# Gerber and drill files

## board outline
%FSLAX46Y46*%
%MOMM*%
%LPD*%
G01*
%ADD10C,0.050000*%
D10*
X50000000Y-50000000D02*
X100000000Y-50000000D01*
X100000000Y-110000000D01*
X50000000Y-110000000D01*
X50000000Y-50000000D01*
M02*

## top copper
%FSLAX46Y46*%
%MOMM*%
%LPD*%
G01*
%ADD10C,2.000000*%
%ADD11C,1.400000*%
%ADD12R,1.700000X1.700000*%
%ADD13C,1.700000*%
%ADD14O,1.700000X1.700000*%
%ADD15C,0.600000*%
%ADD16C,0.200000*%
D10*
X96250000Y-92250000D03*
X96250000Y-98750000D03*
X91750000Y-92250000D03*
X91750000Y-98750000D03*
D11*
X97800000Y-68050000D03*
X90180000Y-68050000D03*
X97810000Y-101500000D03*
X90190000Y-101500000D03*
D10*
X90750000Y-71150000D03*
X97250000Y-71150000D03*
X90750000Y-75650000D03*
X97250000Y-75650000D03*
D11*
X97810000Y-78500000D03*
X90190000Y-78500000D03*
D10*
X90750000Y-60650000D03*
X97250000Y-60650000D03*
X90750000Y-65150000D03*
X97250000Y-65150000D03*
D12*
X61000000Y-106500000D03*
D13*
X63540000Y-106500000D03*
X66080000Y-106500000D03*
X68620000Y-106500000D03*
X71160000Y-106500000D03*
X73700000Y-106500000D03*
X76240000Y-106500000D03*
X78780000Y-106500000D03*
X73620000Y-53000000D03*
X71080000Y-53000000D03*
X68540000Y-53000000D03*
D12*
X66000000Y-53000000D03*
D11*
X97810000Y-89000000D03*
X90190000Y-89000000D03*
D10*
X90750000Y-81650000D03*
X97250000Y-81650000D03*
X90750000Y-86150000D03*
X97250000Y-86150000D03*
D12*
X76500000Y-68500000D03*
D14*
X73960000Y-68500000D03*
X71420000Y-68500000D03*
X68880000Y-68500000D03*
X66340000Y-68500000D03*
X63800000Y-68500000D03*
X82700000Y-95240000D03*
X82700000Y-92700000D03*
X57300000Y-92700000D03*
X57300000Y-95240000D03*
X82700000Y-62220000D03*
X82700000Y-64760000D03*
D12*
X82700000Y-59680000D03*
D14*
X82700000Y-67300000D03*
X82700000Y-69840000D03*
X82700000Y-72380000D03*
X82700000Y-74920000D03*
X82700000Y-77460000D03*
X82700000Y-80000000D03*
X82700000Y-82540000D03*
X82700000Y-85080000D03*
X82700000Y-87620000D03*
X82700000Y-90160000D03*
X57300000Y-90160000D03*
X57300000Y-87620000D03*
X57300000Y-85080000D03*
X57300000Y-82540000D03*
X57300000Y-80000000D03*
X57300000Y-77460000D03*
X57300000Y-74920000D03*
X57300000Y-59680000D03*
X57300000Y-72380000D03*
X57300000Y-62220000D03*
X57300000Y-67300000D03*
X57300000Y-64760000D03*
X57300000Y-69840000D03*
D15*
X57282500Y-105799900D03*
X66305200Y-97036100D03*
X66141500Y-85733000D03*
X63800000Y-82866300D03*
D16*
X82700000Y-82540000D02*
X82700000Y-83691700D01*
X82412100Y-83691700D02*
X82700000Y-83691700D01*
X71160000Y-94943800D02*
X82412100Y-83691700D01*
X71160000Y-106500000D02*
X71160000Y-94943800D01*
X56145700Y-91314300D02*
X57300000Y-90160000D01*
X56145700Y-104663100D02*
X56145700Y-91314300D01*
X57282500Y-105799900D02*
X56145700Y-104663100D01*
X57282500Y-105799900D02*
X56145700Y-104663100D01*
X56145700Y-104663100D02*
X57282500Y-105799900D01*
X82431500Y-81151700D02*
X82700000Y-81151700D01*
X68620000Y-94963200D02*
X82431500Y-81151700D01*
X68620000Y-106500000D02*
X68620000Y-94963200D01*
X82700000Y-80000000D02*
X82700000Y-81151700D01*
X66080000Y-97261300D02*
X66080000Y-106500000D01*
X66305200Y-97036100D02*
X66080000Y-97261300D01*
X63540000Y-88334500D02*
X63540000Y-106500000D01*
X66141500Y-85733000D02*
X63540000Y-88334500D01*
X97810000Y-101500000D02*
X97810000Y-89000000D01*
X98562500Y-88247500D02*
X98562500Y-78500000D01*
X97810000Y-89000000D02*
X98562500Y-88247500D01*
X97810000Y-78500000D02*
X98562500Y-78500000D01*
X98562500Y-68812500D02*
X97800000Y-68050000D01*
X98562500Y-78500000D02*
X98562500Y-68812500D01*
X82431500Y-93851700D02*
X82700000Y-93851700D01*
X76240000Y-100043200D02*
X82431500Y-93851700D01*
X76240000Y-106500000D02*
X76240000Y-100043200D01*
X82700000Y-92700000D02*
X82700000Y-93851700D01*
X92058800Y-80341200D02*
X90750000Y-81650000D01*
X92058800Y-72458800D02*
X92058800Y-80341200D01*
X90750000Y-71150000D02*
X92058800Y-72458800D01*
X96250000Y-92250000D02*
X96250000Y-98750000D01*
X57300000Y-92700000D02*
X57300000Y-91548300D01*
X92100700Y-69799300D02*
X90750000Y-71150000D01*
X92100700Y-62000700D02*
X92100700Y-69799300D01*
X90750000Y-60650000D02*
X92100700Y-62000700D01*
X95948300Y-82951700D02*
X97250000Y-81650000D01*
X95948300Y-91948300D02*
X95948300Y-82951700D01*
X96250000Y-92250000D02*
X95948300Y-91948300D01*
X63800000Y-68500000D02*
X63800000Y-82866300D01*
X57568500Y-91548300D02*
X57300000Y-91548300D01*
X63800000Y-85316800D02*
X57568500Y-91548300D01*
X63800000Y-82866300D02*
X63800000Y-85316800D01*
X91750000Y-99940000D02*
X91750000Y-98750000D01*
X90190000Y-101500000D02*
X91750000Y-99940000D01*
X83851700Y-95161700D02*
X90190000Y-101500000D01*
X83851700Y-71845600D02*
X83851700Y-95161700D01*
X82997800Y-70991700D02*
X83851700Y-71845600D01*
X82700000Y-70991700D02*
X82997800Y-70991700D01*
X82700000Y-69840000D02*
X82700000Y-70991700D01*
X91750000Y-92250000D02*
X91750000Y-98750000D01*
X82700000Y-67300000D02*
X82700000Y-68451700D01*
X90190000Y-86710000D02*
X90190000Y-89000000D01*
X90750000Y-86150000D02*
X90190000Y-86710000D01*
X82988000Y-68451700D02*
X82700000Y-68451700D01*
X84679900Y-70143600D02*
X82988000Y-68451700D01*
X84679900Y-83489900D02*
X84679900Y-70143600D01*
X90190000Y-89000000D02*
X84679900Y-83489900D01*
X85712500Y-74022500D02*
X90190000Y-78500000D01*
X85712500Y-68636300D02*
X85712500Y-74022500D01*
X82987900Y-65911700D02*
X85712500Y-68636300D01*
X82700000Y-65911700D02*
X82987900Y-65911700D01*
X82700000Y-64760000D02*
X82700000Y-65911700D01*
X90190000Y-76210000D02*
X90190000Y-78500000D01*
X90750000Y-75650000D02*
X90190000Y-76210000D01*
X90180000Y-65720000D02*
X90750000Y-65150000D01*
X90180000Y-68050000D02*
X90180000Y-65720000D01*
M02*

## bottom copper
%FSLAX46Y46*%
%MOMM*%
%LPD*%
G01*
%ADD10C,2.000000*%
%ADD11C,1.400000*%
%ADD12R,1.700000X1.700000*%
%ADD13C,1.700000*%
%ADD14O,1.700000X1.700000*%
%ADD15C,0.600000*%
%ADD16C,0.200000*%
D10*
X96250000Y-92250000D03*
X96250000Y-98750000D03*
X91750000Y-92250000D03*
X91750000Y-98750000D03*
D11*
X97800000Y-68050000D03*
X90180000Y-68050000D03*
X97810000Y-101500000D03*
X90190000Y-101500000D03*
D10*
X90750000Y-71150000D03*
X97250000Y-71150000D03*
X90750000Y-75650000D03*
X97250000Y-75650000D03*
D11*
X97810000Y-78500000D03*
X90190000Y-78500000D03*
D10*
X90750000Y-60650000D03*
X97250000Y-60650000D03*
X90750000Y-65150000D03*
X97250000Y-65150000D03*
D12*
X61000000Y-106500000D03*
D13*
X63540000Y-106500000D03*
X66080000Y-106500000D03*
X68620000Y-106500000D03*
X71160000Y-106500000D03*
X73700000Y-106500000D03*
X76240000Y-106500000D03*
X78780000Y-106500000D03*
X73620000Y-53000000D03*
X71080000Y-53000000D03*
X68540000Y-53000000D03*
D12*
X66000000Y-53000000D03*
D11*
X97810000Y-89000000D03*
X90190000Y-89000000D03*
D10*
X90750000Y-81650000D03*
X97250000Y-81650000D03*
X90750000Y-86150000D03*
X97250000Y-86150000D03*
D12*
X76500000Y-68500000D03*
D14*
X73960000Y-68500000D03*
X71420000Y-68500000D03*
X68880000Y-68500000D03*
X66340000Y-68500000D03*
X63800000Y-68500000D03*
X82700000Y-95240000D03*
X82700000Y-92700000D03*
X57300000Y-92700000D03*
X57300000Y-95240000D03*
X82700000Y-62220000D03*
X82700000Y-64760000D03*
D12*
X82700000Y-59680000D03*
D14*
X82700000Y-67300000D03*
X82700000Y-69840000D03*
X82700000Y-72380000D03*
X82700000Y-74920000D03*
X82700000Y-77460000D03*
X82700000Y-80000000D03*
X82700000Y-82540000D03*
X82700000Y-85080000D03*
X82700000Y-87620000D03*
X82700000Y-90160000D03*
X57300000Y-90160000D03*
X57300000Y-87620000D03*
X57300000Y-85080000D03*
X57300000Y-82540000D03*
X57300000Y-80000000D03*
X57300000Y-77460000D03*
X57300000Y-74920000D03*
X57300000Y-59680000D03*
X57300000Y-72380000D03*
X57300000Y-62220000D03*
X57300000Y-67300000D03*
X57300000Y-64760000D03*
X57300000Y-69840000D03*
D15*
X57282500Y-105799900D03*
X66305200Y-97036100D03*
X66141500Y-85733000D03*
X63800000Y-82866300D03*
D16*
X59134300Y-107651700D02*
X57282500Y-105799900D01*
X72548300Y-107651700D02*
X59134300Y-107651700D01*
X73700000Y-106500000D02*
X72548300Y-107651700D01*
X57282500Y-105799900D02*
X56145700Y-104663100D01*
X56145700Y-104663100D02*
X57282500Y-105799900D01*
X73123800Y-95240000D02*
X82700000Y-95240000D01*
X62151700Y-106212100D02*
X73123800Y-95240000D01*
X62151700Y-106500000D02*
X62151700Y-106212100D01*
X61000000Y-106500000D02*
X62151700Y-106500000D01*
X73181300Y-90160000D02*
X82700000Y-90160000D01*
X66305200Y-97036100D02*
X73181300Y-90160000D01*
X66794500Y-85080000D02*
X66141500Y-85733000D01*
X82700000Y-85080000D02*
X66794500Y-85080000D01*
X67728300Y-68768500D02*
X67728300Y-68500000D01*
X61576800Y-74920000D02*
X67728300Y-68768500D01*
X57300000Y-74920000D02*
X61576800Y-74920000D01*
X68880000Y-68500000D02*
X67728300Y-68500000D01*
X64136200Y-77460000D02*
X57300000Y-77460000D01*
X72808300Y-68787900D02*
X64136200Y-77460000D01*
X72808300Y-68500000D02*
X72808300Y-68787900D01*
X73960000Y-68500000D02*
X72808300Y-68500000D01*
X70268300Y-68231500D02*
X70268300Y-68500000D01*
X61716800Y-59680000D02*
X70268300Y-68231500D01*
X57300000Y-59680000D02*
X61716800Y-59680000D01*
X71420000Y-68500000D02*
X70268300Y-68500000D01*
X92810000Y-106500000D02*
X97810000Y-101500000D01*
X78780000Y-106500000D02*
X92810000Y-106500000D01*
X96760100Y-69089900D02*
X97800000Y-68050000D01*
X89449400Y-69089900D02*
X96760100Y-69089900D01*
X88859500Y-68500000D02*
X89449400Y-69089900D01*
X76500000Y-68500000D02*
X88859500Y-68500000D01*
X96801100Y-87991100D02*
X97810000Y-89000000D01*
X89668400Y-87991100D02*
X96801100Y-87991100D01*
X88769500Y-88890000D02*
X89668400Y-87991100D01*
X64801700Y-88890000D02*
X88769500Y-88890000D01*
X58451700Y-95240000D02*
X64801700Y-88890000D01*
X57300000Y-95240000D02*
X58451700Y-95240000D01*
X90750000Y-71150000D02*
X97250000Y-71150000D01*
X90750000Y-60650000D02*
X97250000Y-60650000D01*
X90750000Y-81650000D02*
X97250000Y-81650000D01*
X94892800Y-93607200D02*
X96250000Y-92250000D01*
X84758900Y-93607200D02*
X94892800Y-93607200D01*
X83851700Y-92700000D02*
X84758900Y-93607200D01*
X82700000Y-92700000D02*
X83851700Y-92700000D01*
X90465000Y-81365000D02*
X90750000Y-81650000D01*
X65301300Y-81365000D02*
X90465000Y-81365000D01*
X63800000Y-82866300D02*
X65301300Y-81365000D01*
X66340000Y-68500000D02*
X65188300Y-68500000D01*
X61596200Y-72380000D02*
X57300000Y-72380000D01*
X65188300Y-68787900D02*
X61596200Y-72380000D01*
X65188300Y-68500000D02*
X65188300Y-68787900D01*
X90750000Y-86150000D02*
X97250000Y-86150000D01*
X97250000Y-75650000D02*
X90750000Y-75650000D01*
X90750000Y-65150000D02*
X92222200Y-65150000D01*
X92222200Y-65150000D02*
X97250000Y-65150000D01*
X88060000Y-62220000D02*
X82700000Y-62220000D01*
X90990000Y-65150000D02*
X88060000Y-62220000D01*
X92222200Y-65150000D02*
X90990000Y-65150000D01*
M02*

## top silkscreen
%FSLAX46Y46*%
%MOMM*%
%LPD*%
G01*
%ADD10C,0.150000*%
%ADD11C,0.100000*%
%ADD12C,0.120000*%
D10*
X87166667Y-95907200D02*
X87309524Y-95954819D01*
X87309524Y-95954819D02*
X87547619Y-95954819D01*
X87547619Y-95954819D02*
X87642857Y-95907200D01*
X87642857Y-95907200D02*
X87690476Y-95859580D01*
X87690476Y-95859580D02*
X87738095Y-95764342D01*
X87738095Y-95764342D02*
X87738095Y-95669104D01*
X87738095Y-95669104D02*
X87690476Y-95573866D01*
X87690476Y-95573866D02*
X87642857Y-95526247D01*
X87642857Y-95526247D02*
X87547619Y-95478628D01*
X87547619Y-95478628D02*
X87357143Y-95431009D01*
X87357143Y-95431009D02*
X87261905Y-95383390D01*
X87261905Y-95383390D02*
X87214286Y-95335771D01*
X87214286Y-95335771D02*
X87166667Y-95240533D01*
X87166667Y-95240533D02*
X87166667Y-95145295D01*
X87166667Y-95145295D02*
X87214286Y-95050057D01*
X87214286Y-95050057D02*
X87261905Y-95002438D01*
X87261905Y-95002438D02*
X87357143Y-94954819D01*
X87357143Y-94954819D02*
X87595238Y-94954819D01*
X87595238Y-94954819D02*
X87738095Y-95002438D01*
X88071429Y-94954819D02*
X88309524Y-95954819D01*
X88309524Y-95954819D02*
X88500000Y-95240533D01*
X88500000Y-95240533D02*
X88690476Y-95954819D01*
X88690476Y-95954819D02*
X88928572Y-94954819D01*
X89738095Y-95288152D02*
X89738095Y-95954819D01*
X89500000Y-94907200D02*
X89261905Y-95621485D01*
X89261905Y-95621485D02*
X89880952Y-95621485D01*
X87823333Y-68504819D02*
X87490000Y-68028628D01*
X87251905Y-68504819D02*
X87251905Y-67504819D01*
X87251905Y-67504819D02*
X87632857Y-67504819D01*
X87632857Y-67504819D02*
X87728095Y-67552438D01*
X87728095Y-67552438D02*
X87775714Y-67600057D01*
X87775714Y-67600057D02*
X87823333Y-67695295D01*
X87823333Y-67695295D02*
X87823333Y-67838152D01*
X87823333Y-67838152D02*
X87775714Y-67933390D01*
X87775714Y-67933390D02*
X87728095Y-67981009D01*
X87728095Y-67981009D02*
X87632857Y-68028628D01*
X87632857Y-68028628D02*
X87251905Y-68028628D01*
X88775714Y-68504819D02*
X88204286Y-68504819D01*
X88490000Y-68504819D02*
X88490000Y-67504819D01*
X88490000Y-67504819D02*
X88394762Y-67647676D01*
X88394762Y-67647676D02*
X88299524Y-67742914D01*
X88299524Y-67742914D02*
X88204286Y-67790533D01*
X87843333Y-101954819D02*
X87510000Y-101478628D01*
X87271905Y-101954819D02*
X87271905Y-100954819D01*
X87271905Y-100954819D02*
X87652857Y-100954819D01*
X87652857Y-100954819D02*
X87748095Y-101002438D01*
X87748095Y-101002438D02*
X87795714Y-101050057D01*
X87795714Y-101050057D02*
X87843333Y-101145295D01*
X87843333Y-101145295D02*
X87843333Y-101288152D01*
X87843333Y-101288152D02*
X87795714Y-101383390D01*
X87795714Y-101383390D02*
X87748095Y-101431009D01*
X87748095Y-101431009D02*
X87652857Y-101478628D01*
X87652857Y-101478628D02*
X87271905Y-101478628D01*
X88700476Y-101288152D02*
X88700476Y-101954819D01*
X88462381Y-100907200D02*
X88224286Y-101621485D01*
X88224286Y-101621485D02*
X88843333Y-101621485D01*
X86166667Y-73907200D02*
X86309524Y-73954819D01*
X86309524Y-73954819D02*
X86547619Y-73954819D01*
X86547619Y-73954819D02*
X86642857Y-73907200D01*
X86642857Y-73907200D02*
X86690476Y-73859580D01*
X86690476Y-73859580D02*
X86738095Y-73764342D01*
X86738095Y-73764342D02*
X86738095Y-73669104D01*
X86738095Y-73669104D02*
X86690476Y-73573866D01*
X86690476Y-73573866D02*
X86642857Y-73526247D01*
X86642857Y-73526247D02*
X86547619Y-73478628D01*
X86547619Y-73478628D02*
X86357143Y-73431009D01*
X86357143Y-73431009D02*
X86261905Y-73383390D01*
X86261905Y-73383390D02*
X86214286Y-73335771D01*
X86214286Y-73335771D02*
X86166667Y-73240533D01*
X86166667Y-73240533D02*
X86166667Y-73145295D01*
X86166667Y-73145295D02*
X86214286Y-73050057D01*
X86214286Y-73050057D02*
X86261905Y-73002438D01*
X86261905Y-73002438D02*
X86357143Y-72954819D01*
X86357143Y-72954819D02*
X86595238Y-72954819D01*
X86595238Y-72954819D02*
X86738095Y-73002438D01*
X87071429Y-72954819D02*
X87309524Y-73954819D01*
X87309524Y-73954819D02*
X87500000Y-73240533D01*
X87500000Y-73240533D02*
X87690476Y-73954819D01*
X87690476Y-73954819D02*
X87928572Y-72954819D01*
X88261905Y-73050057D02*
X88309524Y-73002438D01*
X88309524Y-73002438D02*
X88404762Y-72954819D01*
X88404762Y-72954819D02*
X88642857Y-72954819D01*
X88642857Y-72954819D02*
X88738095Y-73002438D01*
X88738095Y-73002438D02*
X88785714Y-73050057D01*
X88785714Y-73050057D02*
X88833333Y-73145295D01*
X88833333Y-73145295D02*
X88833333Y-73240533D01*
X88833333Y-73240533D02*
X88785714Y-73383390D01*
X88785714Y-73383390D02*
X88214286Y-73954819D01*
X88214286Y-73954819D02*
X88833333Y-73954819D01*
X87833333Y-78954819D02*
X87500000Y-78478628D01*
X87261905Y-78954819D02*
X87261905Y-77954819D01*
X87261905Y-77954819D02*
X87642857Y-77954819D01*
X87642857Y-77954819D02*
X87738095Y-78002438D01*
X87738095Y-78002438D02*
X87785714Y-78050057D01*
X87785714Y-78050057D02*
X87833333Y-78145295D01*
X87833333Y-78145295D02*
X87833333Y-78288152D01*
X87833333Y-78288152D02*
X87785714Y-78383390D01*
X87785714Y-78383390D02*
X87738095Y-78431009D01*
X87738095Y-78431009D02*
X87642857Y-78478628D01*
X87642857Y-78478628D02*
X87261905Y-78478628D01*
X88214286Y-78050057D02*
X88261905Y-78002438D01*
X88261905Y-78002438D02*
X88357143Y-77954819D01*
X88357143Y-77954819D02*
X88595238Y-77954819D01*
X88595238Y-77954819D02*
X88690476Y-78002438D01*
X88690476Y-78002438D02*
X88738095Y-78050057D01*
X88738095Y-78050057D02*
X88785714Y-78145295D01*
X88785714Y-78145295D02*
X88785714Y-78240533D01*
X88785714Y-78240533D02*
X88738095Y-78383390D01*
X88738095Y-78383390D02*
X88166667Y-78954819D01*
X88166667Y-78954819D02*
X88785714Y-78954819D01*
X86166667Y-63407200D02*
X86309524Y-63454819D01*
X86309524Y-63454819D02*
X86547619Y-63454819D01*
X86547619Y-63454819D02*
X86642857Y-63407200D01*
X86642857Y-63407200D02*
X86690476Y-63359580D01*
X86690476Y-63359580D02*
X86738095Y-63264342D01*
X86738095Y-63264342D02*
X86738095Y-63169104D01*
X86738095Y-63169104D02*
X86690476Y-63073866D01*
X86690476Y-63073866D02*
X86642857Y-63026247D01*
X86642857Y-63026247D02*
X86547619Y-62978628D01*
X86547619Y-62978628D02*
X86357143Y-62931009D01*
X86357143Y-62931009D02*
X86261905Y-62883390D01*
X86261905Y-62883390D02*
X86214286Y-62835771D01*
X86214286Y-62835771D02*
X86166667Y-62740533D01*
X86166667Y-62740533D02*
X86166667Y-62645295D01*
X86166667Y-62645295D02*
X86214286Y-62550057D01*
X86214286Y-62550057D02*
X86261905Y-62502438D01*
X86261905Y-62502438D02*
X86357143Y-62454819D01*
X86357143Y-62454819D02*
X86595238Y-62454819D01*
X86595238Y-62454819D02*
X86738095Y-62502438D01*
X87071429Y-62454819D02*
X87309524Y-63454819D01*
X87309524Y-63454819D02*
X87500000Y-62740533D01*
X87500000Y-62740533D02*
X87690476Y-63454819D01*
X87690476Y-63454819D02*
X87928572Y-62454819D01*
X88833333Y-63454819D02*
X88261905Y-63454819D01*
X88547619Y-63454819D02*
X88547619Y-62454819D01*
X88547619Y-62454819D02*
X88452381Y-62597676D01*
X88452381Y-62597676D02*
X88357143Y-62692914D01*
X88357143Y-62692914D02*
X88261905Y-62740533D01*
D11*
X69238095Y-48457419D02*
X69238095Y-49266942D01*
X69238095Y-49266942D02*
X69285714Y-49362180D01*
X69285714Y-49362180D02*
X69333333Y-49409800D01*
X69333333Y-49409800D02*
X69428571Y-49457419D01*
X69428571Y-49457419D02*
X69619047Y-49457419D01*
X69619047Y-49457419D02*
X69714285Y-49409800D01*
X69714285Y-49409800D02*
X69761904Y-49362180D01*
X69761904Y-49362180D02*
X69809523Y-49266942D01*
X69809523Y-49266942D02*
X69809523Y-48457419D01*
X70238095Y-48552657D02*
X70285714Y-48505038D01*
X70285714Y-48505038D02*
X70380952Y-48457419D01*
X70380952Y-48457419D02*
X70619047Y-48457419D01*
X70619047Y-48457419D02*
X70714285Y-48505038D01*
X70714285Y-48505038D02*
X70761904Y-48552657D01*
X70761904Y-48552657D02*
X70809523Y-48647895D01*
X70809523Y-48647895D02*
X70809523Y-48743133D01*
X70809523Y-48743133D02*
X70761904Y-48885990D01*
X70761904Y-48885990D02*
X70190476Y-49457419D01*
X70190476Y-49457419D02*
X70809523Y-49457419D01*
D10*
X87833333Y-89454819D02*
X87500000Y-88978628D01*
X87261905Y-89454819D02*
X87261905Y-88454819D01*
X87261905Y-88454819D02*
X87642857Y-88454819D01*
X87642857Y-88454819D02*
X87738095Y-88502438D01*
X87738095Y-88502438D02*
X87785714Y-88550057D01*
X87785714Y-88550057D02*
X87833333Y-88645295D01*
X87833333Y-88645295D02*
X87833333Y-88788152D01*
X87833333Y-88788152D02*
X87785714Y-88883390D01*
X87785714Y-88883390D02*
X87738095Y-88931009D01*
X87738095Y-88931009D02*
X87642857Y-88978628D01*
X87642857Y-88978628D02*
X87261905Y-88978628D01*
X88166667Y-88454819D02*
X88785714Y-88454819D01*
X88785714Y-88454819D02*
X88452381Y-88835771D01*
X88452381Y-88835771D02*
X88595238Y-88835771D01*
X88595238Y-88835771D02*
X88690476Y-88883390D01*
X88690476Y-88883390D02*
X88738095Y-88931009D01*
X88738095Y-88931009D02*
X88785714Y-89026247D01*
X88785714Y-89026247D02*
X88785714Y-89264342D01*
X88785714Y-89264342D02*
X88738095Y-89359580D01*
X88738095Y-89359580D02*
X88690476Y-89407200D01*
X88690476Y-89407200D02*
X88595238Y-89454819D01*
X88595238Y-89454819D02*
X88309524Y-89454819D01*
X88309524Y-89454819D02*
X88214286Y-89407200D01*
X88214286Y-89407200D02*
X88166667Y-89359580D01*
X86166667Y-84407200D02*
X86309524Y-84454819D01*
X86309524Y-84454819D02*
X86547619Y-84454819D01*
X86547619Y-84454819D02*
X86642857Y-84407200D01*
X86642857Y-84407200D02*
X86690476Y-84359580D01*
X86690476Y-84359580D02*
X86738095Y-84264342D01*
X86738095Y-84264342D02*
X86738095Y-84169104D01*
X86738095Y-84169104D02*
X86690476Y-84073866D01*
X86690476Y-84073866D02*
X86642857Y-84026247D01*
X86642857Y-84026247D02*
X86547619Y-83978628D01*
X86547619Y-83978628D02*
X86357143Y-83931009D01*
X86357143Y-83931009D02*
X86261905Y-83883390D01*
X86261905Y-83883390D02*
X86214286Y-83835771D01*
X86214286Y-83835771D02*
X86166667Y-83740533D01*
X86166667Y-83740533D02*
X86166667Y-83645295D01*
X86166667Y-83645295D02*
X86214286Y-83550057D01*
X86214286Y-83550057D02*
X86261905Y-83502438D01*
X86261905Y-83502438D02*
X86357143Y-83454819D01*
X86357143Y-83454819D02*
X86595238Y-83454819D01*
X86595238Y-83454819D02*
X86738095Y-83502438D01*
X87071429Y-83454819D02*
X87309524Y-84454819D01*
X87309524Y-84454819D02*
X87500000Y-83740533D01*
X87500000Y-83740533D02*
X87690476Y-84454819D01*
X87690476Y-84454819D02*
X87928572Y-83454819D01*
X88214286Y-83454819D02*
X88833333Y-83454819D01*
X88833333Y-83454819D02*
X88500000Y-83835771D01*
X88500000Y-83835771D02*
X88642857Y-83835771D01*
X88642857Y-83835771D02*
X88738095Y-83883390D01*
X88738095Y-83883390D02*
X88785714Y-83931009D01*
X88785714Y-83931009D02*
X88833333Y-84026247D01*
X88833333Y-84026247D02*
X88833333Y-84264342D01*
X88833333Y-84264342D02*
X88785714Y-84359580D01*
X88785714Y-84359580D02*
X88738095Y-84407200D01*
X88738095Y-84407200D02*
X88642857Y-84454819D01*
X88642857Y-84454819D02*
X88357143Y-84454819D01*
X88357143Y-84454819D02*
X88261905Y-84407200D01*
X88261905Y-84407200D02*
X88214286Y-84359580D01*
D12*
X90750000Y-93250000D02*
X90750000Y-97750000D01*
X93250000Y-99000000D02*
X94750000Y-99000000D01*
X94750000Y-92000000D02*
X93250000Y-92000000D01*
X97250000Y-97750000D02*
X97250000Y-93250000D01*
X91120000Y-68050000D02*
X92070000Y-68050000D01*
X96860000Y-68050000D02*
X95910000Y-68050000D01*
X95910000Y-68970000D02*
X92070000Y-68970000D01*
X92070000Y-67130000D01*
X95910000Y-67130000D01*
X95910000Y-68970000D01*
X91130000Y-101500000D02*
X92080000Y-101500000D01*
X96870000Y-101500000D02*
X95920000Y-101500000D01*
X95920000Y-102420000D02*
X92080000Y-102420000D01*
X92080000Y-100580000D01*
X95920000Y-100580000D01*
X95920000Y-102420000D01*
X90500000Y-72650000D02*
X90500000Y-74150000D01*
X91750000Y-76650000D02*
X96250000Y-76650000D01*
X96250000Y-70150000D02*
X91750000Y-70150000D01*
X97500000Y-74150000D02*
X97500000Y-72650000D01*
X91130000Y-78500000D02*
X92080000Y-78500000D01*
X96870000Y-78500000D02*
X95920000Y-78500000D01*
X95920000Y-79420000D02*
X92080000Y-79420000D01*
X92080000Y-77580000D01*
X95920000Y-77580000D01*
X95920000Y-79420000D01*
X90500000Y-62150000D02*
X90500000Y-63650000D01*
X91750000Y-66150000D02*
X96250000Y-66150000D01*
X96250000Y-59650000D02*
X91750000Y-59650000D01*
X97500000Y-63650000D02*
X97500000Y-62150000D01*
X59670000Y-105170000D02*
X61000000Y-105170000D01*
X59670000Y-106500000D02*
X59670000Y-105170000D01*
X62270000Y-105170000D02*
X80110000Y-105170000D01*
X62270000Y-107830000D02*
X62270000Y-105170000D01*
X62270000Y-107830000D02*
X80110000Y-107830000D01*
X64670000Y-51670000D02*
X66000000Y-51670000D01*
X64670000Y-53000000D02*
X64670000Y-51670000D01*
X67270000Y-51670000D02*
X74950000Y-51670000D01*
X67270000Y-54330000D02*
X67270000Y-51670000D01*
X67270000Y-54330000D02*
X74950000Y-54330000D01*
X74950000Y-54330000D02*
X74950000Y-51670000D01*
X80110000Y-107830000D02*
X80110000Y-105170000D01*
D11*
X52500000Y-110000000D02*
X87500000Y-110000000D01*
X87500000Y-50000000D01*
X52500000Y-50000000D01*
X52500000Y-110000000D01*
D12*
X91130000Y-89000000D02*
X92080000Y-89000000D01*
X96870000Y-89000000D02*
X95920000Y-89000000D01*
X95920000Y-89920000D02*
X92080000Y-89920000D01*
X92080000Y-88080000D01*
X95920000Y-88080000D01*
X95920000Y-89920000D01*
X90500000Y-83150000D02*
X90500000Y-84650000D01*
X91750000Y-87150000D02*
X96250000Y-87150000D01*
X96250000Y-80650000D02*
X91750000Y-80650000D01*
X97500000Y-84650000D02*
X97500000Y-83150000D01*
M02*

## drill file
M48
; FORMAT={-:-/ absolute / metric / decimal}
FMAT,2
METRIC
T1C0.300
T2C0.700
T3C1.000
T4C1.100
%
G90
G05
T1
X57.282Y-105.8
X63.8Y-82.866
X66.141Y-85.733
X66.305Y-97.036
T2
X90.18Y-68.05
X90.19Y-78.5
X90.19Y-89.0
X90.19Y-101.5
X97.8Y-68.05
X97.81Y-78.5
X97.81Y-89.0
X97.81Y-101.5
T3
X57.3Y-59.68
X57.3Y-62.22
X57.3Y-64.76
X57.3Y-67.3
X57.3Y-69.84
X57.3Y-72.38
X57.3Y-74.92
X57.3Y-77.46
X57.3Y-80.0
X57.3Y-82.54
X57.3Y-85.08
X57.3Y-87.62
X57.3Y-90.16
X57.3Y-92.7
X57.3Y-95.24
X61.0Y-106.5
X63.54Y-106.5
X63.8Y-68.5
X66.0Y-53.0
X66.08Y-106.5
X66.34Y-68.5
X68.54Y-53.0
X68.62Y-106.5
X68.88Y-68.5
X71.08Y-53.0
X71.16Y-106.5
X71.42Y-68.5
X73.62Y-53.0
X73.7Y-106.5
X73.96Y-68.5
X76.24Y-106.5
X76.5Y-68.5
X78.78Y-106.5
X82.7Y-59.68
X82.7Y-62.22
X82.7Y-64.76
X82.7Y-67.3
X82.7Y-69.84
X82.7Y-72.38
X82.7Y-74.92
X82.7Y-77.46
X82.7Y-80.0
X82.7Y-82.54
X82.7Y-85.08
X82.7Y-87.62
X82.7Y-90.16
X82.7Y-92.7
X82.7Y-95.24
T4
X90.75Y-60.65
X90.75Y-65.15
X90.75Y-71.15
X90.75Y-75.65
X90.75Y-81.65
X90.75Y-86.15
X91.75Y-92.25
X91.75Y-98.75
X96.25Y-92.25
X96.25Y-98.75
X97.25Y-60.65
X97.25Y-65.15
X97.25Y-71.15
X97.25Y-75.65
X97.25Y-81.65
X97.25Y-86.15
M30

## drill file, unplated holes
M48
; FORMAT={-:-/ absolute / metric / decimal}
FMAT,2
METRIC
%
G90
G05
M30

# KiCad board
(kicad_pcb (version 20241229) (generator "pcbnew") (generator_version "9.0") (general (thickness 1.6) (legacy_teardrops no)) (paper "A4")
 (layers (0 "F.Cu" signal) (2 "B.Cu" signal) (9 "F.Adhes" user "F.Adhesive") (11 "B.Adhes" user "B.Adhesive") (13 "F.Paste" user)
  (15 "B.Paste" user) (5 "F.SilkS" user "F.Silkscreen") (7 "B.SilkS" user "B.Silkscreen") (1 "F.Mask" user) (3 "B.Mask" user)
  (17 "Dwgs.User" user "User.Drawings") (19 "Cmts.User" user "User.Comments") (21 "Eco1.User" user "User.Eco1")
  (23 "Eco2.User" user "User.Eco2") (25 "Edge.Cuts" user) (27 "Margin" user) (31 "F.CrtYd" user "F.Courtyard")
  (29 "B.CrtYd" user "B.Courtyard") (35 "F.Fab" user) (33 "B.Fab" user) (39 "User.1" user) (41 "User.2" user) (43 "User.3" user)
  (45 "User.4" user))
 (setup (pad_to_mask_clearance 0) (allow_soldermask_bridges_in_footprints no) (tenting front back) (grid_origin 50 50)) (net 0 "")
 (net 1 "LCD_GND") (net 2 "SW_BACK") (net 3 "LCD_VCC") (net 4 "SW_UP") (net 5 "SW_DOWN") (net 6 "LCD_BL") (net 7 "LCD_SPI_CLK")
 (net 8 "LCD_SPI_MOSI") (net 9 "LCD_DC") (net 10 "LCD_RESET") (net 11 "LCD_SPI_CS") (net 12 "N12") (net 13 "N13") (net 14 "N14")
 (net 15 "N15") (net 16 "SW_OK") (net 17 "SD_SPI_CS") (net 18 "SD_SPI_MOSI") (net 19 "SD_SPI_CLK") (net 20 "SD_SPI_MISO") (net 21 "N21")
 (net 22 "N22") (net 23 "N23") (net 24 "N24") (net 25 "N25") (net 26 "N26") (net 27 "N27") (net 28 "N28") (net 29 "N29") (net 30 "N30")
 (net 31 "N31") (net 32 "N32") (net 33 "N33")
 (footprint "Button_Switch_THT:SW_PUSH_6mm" (layer "F.Cu") (at 96.25 92.25 -90)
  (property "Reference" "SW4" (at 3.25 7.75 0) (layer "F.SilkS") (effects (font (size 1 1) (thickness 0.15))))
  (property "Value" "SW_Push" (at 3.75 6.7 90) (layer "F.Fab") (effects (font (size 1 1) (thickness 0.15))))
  (fp_line (start 1 5.5) (end 5.5 5.5) (stroke (width 0.12) (type solid)) (layer "F.SilkS"))
  (fp_line (start 6.75 3) (end 6.75 1.5) (stroke (width 0.12) (type solid)) (layer "F.SilkS"))
  (fp_line (start -0.25 1.5) (end -0.25 3) (stroke (width 0.12) (type solid)) (layer "F.SilkS"))
  (fp_line (start 5.5 -1) (end 1 -1) (stroke (width 0.12) (type solid)) (layer "F.SilkS"))
  (pad "1" thru_hole circle (at 0 0) (size 2 2) (drill 1.1) (layers "*.Cu" "*.Mask") (remove_unused_layers no) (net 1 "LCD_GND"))
  (pad "1" thru_hole circle (at 6.5 0) (size 2 2) (drill 1.1) (layers "*.Cu" "*.Mask") (remove_unused_layers no) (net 1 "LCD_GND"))
  (pad "2" thru_hole circle (at 0 4.5) (size 2 2) (drill 1.1) (layers "*.Cu" "*.Mask") (remove_unused_layers no) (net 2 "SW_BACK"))
  (pad "2" thru_hole circle (at 6.5 4.5) (size 2 2) (drill 1.1) (layers "*.Cu" "*.Mask") (remove_unused_layers no) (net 2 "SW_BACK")))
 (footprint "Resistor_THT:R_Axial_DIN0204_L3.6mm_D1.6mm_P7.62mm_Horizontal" (layer "F.Cu") (at 97.8 68.05 180)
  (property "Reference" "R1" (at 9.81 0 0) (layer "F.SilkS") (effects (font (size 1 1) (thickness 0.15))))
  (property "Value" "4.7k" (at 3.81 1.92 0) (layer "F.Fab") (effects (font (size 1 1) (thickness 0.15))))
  (fp_line (start 6.68 0) (end 5.73 0) (stroke (width 0.12) (type solid)) (layer "F.SilkS"))
  (fp_line (start 0.94 0) (end 1.89 0) (stroke (width 0.12) (type solid)) (layer "F.SilkS"))
  (fp_rect (start 1.89 -0.92) (end 5.73 0.92) (stroke (width 0.12) (type solid)) (fill no) (layer "F.SilkS"))
  (pad "1" thru_hole circle (at 0 0 180) (size 1.4 1.4) (drill 0.7) (layers "*.Cu" "*.Mask") (remove_unused_layers no) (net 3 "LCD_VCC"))
  (pad "2" thru_hole circle (at 7.62 0 180) (size 1.4 1.4) (drill 0.7) (layers "*.Cu" "*.Mask") (remove_unused_layers no) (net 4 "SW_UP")))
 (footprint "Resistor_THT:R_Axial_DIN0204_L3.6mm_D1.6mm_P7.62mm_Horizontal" (layer "F.Cu") (at 97.81 101.5 180)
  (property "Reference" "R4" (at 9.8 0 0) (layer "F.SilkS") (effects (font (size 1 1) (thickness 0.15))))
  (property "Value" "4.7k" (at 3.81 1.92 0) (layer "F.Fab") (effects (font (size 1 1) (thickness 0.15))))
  (fp_line (start 6.68 0) (end 5.73 0) (stroke (width 0.12) (type solid)) (layer "F.SilkS"))
  (fp_line (start 0.94 0) (end 1.89 0) (stroke (width 0.12) (type solid)) (layer "F.SilkS"))
  (fp_rect (start 1.89 -0.92) (end 5.73 0.92) (stroke (width 0.12) (type solid)) (fill no) (layer "F.SilkS"))
  (pad "1" thru_hole circle (at 0 0 180) (size 1.4 1.4) (drill 0.7) (layers "*.Cu" "*.Mask") (remove_unused_layers no) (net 3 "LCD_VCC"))
  (pad "2" thru_hole circle (at 7.62 0 180) (size 1.4 1.4) (drill 0.7) (layers "*.Cu" "*.Mask") (remove_unused_layers no) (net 2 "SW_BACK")))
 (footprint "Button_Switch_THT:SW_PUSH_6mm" (layer "F.Cu") (at 90.75 71.15)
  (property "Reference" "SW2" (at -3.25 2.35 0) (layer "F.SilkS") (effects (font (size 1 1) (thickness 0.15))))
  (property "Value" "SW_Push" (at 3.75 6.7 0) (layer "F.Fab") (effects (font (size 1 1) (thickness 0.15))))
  (fp_line (start -0.25 1.5) (end -0.25 3) (stroke (width 0.12) (type solid)) (layer "F.SilkS"))
  (fp_line (start 1 5.5) (end 5.5 5.5) (stroke (width 0.12) (type solid)) (layer "F.SilkS"))
  (fp_line (start 5.5 -1) (end 1 -1) (stroke (width 0.12) (type solid)) (layer "F.SilkS"))
  (fp_line (start 6.75 3) (end 6.75 1.5) (stroke (width 0.12) (type solid)) (layer "F.SilkS"))
  (pad "1" thru_hole circle (at 0 0 90) (size 2 2) (drill 1.1) (layers "*.Cu" "*.Mask") (remove_unused_layers no) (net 1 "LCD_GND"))
  (pad "1" thru_hole circle (at 6.5 0 90) (size 2 2) (drill 1.1) (layers "*.Cu" "*.Mask") (remove_unused_layers no) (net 1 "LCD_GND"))
  (pad "2" thru_hole circle (at 0 4.5 90) (size 2 2) (drill 1.1) (layers "*.Cu" "*.Mask") (remove_unused_layers no) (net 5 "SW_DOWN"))
  (pad "2" thru_hole circle (at 6.5 4.5 90) (size 2 2) (drill 1.1) (layers "*.Cu" "*.Mask") (remove_unused_layers no) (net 5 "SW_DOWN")))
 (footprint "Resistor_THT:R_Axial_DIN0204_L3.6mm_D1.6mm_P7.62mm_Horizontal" (layer "F.Cu") (at 97.81 78.5 180)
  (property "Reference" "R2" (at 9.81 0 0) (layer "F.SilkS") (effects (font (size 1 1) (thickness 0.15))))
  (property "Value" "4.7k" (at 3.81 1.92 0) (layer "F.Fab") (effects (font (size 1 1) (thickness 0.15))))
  (fp_line (start 6.68 0) (end 5.73 0) (stroke (width 0.12) (type solid)) (layer "F.SilkS"))
  (fp_line (start 0.94 0) (end 1.89 0) (stroke (width 0.12) (type solid)) (layer "F.SilkS"))
  (fp_rect (start 1.89 -0.92) (end 5.73 0.92) (stroke (width 0.12) (type solid)) (fill no) (layer "F.SilkS"))
  (pad "1" thru_hole circle (at 0 0 180) (size 1.4 1.4) (drill 0.7) (layers "*.Cu" "*.Mask") (remove_unused_layers no) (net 3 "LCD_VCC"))
  (pad "2" thru_hole circle (at 7.62 0 180) (size 1.4 1.4) (drill 0.7) (layers "*.Cu" "*.Mask") (remove_unused_layers no) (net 5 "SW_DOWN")))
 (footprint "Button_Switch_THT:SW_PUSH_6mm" (layer "F.Cu") (at 90.75 60.65)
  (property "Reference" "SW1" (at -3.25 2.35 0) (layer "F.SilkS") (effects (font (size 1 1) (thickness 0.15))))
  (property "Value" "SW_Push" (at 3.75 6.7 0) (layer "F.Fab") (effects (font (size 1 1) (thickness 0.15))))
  (fp_line (start -0.25 1.5) (end -0.25 3) (stroke (width 0.12) (type solid)) (layer "F.SilkS"))
  (fp_line (start 1 5.5) (end 5.5 5.5) (stroke (width 0.12) (type solid)) (layer "F.SilkS"))
  (fp_line (start 5.5 -1) (end 1 -1) (stroke (width 0.12) (type solid)) (layer "F.SilkS"))
  (fp_line (start 6.75 3) (end 6.75 1.5) (stroke (width 0.12) (type solid)) (layer "F.SilkS"))
  (pad "1" thru_hole circle (at 0 0 90) (size 2 2) (drill 1.1) (layers "*.Cu" "*.Mask") (remove_unused_layers no) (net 1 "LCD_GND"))
  (pad "1" thru_hole circle (at 6.5 0 90) (size 2 2) (drill 1.1) (layers "*.Cu" "*.Mask") (remove_unused_layers no) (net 1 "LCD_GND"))
  (pad "2" thru_hole circle (at 0 4.5 90) (size 2 2) (drill 1.1) (layers "*.Cu" "*.Mask") (remove_unused_layers no) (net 4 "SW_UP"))
  (pad "2" thru_hole circle (at 6.5 4.5 90) (size 2 2) (drill 1.1) (layers "*.Cu" "*.Mask") (remove_unused_layers no) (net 4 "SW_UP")))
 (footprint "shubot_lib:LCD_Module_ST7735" (layer "F.Cu") (at 70 80 90)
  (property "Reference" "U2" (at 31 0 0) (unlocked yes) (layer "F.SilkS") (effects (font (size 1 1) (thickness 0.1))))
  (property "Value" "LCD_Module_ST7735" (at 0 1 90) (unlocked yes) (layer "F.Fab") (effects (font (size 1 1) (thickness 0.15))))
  (fp_line (start -25.17 -10.33) (end -25.17 -9) (stroke (width 0.12) (type solid)) (layer "F.SilkS"))
  (fp_line (start -26.5 -10.33) (end -25.17 -10.33) (stroke (width 0.12) (type solid)) (layer "F.SilkS"))
  (fp_line (start -25.17 -7.73) (end -25.17 10.11) (stroke (width 0.12) (type solid)) (layer "F.SilkS"))
  (fp_line (start -27.83 -7.73) (end -25.17 -7.73) (stroke (width 0.12) (type solid)) (layer "F.SilkS"))
  (fp_line (start -27.83 -7.73) (end -27.83 10.11) (stroke (width 0.12) (type solid)) (layer "F.SilkS"))
  (fp_line (start 28.33 -5.33) (end 28.33 -4) (stroke (width 0.12) (type solid)) (layer "F.SilkS"))
  (fp_line (start 27 -5.33) (end 28.33 -5.33) (stroke (width 0.12) (type solid)) (layer "F.SilkS"))
  (fp_line (start 28.33 -2.73) (end 28.33 4.95) (stroke (width 0.12) (type solid)) (layer "F.SilkS"))
  (fp_line (start 25.67 -2.73) (end 28.33 -2.73) (stroke (width 0.12) (type solid)) (layer "F.SilkS"))
  (fp_line (start 25.67 -2.73) (end 25.67 4.95) (stroke (width 0.12) (type solid)) (layer "F.SilkS"))
  (fp_line (start 25.67 4.95) (end 28.33 4.95) (stroke (width 0.12) (type solid)) (layer "F.SilkS"))
  (fp_line (start -27.83 10.11) (end -25.17 10.11) (stroke (width 0.12) (type solid)) (layer "F.SilkS"))
  (fp_rect (start -30 -17.5) (end 30 17.5) (stroke (width 0.1) (type default)) (fill no) (layer "F.SilkS"))
  (pad "1" thru_hole rect (at -26.5 -9 90) (size 1.7 1.7) (drill 1) (layers "*.Cu" "*.Mask") (remove_unused_layers no) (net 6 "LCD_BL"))
  (pad "2" thru_hole circle (at -26.5 -6.46 90) (size 1.7 1.7) (drill 1) (layers "*.Cu" "*.Mask") (remove_unused_layers no)
   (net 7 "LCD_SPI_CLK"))
  (pad "3" thru_hole circle (at -26.5 -3.92 90) (size 1.7 1.7) (drill 1) (layers "*.Cu" "*.Mask") (remove_unused_layers no)
   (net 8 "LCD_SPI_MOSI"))
  (pad "4" thru_hole circle (at -26.5 -1.38 90) (size 1.7 1.7) (drill 1) (layers "*.Cu" "*.Mask") (remove_unused_layers no) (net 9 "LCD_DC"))
  (pad "5" thru_hole circle (at -26.5 1.16 90) (size 1.7 1.7) (drill 1) (layers "*.Cu" "*.Mask") (remove_unused_layers no)
   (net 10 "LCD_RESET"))
  (pad "6" thru_hole circle (at -26.5 3.7 90) (size 1.7 1.7) (drill 1) (layers "*.Cu" "*.Mask") (remove_unused_layers no)
   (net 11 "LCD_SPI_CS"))
  (pad "7" thru_hole circle (at -26.5 6.24 90) (size 1.7 1.7) (drill 1) (layers "*.Cu" "*.Mask") (remove_unused_layers no) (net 1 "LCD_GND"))
  (pad "8" thru_hole circle (at -26.5 8.78 90) (size 1.7 1.7) (drill 1) (layers "*.Cu" "*.Mask") (remove_unused_layers no) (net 3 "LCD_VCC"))
  (pad "9" thru_hole circle (at 27 3.62 90) (size 1.7 1.7) (drill 1) (layers "*.Cu" "*.Mask") (remove_unused_layers no) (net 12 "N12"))
  (pad "10" thru_hole circle (at 27 1.08 90) (size 1.7 1.7) (drill 1) (layers "*.Cu" "*.Mask") (remove_unused_layers no) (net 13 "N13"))
  (pad "11" thru_hole circle (at 27 -1.46 90) (size 1.7 1.7) (drill 1) (layers "*.Cu" "*.Mask") (remove_unused_layers no) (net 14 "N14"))
  (pad "12" thru_hole rect (at 27 -4 90) (size 1.7 1.7) (drill 1) (layers "*.Cu" "*.Mask") (remove_unused_layers no) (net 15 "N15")))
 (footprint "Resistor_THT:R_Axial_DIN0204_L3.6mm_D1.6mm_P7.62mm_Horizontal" (layer "F.Cu") (at 97.81 89 180)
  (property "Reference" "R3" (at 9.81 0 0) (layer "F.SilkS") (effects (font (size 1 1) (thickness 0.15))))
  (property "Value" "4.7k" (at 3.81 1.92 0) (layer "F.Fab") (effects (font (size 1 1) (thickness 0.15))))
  (fp_line (start 6.68 0) (end 5.73 0) (stroke (width 0.12) (type solid)) (layer "F.SilkS"))
  (fp_line (start 0.94 0) (end 1.89 0) (stroke (width 0.12) (type solid)) (layer "F.SilkS"))
  (fp_rect (start 1.89 -0.92) (end 5.73 0.92) (stroke (width 0.12) (type solid)) (fill no) (layer "F.SilkS"))
  (pad "1" thru_hole circle (at 0 0 180) (size 1.4 1.4) (drill 0.7) (layers "*.Cu" "*.Mask") (remove_unused_layers no) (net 3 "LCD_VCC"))
  (pad "2" thru_hole circle (at 7.62 0 180) (size 1.4 1.4) (drill 0.7) (layers "*.Cu" "*.Mask") (remove_unused_layers no) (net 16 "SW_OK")))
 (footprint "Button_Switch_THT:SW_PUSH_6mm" (layer "F.Cu") (at 90.75 81.65)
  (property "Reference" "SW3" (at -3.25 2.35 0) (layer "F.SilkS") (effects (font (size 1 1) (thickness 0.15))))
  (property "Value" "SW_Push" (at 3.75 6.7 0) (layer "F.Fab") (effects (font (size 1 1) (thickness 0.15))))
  (fp_line (start -0.25 1.5) (end -0.25 3) (stroke (width 0.12) (type solid)) (layer "F.SilkS"))
  (fp_line (start 1 5.5) (end 5.5 5.5) (stroke (width 0.12) (type solid)) (layer "F.SilkS"))
  (fp_line (start 5.5 -1) (end 1 -1) (stroke (width 0.12) (type solid)) (layer "F.SilkS"))
  (fp_line (start 6.75 3) (end 6.75 1.5) (stroke (width 0.12) (type solid)) (layer "F.SilkS"))
  (pad "1" thru_hole circle (at 0 0 90) (size 2 2) (drill 1.1) (layers "*.Cu" "*.Mask") (remove_unused_layers no) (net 1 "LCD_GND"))
  (pad "1" thru_hole circle (at 6.5 0 90) (size 2 2) (drill 1.1) (layers "*.Cu" "*.Mask") (remove_unused_layers no) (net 1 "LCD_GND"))
  (pad "2" thru_hole circle (at 0 4.5 90) (size 2 2) (drill 1.1) (layers "*.Cu" "*.Mask") (remove_unused_layers no) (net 16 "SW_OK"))
  (pad "2" thru_hole circle (at 6.5 4.5 90) (size 2 2) (drill 1.1) (layers "*.Cu" "*.Mask") (remove_unused_layers no) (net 16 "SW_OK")))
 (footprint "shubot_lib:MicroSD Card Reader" (layer "B.Cu") (at 76.5 68.5 90)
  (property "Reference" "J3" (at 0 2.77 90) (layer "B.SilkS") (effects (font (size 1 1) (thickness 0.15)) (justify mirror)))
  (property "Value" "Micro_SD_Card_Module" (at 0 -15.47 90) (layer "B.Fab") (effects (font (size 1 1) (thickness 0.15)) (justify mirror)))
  (pad "1" thru_hole rect (at 0 0 90) (size 1.7 1.7) (drill 1) (layers "*.Cu" "*.Mask") (remove_unused_layers no) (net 3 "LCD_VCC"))
  (pad "2" thru_hole oval (at 0 -2.54 90) (size 1.7 1.7) (drill 1) (layers "*.Cu" "*.Mask") (remove_unused_layers no) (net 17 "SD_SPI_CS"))
  (pad "3" thru_hole oval (at 0 -5.08 90) (size 1.7 1.7) (drill 1) (layers "*.Cu" "*.Mask") (remove_unused_layers no) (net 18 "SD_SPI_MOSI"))
  (pad "4" thru_hole oval (at 0 -7.62 90) (size 1.7 1.7) (drill 1) (layers "*.Cu" "*.Mask") (remove_unused_layers no) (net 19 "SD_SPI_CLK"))
  (pad "5" thru_hole oval (at 0 -10.16 90) (size 1.7 1.7) (drill 1) (layers "*.Cu" "*.Mask") (remove_unused_layers no)
   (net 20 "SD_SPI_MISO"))
  (pad "6" thru_hole oval (at 0 -12.7 90) (size 1.7 1.7) (drill 1) (layers "*.Cu" "*.Mask") (remove_unused_layers no) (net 1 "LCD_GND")))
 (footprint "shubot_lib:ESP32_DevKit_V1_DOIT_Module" (layer "B.Cu") (at 70 80 180)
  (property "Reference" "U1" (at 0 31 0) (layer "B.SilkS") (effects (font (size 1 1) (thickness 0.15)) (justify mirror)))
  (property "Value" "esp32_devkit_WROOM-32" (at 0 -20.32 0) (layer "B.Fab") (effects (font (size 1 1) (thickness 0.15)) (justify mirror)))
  (pad "1" thru_hole oval (at -12.7 -15.24 180) (size 1.7 1.7) (drill 1) (layers "*.Cu" "*.Mask") (remove_unused_layers no) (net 6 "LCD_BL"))
  (pad "2" thru_hole oval (at -12.7 -12.7 180) (size 1.7 1.7) (drill 1) (layers "*.Cu" "*.Mask") (remove_unused_layers no) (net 1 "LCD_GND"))
  (pad "2" thru_hole oval (at 12.7 -12.7 180) (size 1.7 1.7) (drill 1) (layers "*.Cu" "*.Mask") (remove_unused_layers no) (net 1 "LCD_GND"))
  (pad "3" thru_hole oval (at 12.7 -15.24 180) (size 1.7 1.7) (drill 1) (layers "*.Cu" "*.Mask") (remove_unused_layers no) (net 3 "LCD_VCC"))
  (pad "5" thru_hole oval (at -12.7 17.78 180) (size 1.7 1.7) (drill 1) (layers "*.Cu" "*.Mask") (remove_unused_layers no) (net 4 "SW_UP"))
  (pad "8" thru_hole oval (at -12.7 15.24 180) (size 1.7 1.7) (drill 1) (layers "*.Cu" "*.Mask") (remove_unused_layers no) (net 5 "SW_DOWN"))
  (pad "9" thru_hole rect (at -12.7 20.32 180) (size 1.7 1.7) (drill 1) (layers "*.Cu" "*.Mask") (remove_unused_layers no) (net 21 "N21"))
  (pad "10" thru_hole oval (at -12.7 12.7 180) (size 1.7 1.7) (drill 1) (layers "*.Cu" "*.Mask") (remove_unused_layers no) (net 16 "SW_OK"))
  (pad "11" thru_hole oval (at -12.7 10.16 180) (size 1.7 1.7) (drill 1) (layers "*.Cu" "*.Mask") (remove_unused_layers no)
   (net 2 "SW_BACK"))
  (pad "12" thru_hole oval (at -12.7 7.62 180) (size 1.7 1.7) (drill 1) (layers "*.Cu" "*.Mask") (remove_unused_layers no) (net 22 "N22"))
  (pad "13" thru_hole oval (at -12.7 5.08 180) (size 1.7 1.7) (drill 1) (layers "*.Cu" "*.Mask") (remove_unused_layers no) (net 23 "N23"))
  (pad "14" thru_hole oval (at -12.7 2.54 180) (size 1.7 1.7) (drill 1) (layers "*.Cu" "*.Mask") (remove_unused_layers no) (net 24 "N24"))
  (pad "15" thru_hole oval (at -12.7 0 180) (size 1.7 1.7) (drill 1) (layers "*.Cu" "*.Mask") (remove_unused_layers no) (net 9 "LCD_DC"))
  (pad "16" thru_hole oval (at -12.7 -2.54 180) (size 1.7 1.7) (drill 1) (layers "*.Cu" "*.Mask") (remove_unused_layers no)
   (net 10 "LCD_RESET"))
  (pad "17" thru_hole oval (at -12.7 -5.08 180) (size 1.7 1.7) (drill 1) (layers "*.Cu" "*.Mask") (remove_unused_layers no)
   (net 7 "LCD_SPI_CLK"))
  (pad "18" thru_hole oval (at -12.7 -7.62 180) (size 1.7 1.7) (drill 1) (layers "*.Cu" "*.Mask") (remove_unused_layers no) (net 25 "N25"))
  (pad "20" thru_hole oval (at -12.7 -10.16 180) (size 1.7 1.7) (drill 1) (layers "*.Cu" "*.Mask") (remove_unused_layers no)
   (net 8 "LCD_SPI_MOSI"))
  (pad "21" thru_hole oval (at 12.7 -10.16 180) (size 1.7 1.7) (drill 1) (layers "*.Cu" "*.Mask") (remove_unused_layers no)
   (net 11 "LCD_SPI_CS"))
  (pad "22" thru_hole oval (at 12.7 -7.62 180) (size 1.7 1.7) (drill 1) (layers "*.Cu" "*.Mask") (remove_unused_layers no) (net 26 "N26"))
  (pad "24" thru_hole oval (at 12.7 -5.08 180) (size 1.7 1.7) (drill 1) (layers "*.Cu" "*.Mask") (remove_unused_layers no) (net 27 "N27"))
  (pad "25" thru_hole oval (at 12.7 -2.54 180) (size 1.7 1.7) (drill 1) (layers "*.Cu" "*.Mask") (remove_unused_layers no) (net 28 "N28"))
  (pad "27" thru_hole oval (at 12.7 0 180) (size 1.7 1.7) (drill 1) (layers "*.Cu" "*.Mask") (remove_unused_layers no) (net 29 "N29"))
  (pad "34" thru_hole oval (at 12.7 2.54 180) (size 1.7 1.7) (drill 1) (layers "*.Cu" "*.Mask") (remove_unused_layers no)
   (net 17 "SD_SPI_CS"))
  (pad "35" thru_hole oval (at 12.7 5.08 180) (size 1.7 1.7) (drill 1) (layers "*.Cu" "*.Mask") (remove_unused_layers no)
   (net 19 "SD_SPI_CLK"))
  (pad "36" thru_hole oval (at 12.7 20.32 180) (size 1.7 1.7) (drill 1) (layers "*.Cu" "*.Mask") (remove_unused_layers no)
   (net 18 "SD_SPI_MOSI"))
  (pad "38" thru_hole oval (at 12.7 7.62 180) (size 1.7 1.7) (drill 1) (layers "*.Cu" "*.Mask") (remove_unused_layers no)
   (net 20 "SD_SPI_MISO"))
  (pad "39" thru_hole oval (at 12.7 17.78 180) (size 1.7 1.7) (drill 1) (layers "*.Cu" "*.Mask") (remove_unused_layers no) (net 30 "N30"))
  (pad "40" thru_hole oval (at 12.7 12.7 180) (size 1.7 1.7) (drill 1) (layers "*.Cu" "*.Mask") (remove_unused_layers no) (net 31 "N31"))
  (pad "41" thru_hole oval (at 12.7 15.24 180) (size 1.7 1.7) (drill 1) (layers "*.Cu" "*.Mask") (remove_unused_layers no) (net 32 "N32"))
  (pad "42" thru_hole oval (at 12.7 10.16 180) (size 1.7 1.7) (drill 1) (layers "*.Cu" "*.Mask") (remove_unused_layers no) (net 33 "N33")))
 (gr_rect (start 50 50) (end 100 110) (stroke (width 0.05) (type default)) (fill no) (layer "Edge.Cuts"))
 (segment (start 90.18 68.05) (end 90.18 65.72) (width 0.2) (layer "F.Cu") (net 4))
 (segment (start 90.18 65.72) (end 90.75 65.15) (width 0.2) (layer "F.Cu") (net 4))
 (segment (start 90.99 65.15) (end 88.06 62.22) (width 0.2) (layer "B.Cu") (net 4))
 (segment (start 90.75 65.15) (end 92.2222 65.15) (width 0.2) (layer "B.Cu") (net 4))
 (segment (start 92.2222 65.15) (end 90.99 65.15) (width 0.2) (layer "B.Cu") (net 4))
 (segment (start 88.06 62.22) (end 82.7 62.22) (width 0.2) (layer "B.Cu") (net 4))
 (segment (start 92.2222 65.15) (end 97.25 65.15) (width 0.2) (layer "B.Cu") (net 4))
 (segment (start 82.9879 65.9117) (end 85.7125 68.6363) (width 0.2) (layer "F.Cu") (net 5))
 (segment (start 85.7125 68.6363) (end 85.7125 74.0225) (width 0.2) (layer "F.Cu") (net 5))
 (segment (start 82.7 65.9117) (end 82.9879 65.9117) (width 0.2) (layer "F.Cu") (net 5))
 (segment (start 90.19 76.21) (end 90.19 78.5) (width 0.2) (layer "F.Cu") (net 5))
 (segment (start 85.7125 74.0225) (end 90.19 78.5) (width 0.2) (layer "F.Cu") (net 5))
 (segment (start 82.7 64.76) (end 82.7 65.9117) (width 0.2) (layer "F.Cu") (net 5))
 (segment (start 90.75 75.65) (end 90.19 76.21) (width 0.2) (layer "F.Cu") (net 5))
 (segment (start 97.25 75.65) (end 90.75 75.65) (width 0.2) (layer "B.Cu") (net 5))
 (segment (start 90.75 86.15) (end 90.19 86.71) (width 0.2) (layer "F.Cu") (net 16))
 (segment (start 90.19 89) (end 84.6799 83.4899) (width 0.2) (layer "F.Cu") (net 16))
 (segment (start 84.6799 83.4899) (end 84.6799 70.1436) (width 0.2) (layer "F.Cu") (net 16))
 (segment (start 82.7 67.3) (end 82.7 68.4517) (width 0.2) (layer "F.Cu") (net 16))
 (segment (start 90.19 86.71) (end 90.19 89) (width 0.2) (layer "F.Cu") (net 16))
 (segment (start 82.988 68.4517) (end 82.7 68.4517) (width 0.2) (layer "F.Cu") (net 16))
 (segment (start 84.6799 70.1436) (end 82.988 68.4517) (width 0.2) (layer "F.Cu") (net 16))
 (segment (start 90.75 86.15) (end 97.25 86.15) (width 0.2) (layer "B.Cu") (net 16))
 (segment (start 83.8517 71.8456) (end 83.8517 95.1617) (width 0.2) (layer "F.Cu") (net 2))
 (segment (start 82.7 70.9917) (end 82.9978 70.9917) (width 0.2) (layer "F.Cu") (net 2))
 (segment (start 90.19 101.5) (end 91.75 99.94) (width 0.2) (layer "F.Cu") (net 2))
 (segment (start 83.8517 95.1617) (end 90.19 101.5) (width 0.2) (layer "F.Cu") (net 2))
 (segment (start 91.75 92.25) (end 91.75 98.75) (width 0.2) (layer "F.Cu") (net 2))
 (segment (start 82.7 69.84) (end 82.7 70.9917) (width 0.2) (layer "F.Cu") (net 2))
 (segment (start 91.75 99.94) (end 91.75 98.75) (width 0.2) (layer "F.Cu") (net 2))
 (segment (start 82.9978 70.9917) (end 83.8517 71.8456) (width 0.2) (layer "F.Cu") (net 2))
 (segment (start 66.34 68.5) (end 65.1883 68.5) (width 0.2) (layer "B.Cu") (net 20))
 (segment (start 65.1883 68.5) (end 65.1883 68.7879) (width 0.2) (layer "B.Cu") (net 20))
 (segment (start 61.5962 72.38) (end 57.3 72.38) (width 0.2) (layer "B.Cu") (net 20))
 (segment (start 65.1883 68.7879) (end 61.5962 72.38) (width 0.2) (layer "B.Cu") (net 20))
 (segment (start 92.1007 69.7993) (end 90.75 71.15) (width 0.2) (layer "F.Cu") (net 1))
 (segment (start 90.75 60.65) (end 92.1007 62.0007) (width 0.2) (layer "F.Cu") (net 1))
 (segment (start 82.4315 93.8517) (end 82.7 93.8517) (width 0.2) (layer "F.Cu") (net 1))
 (segment (start 92.1007 62.0007) (end 92.1007 69.7993) (width 0.2) (layer "F.Cu") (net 1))
 (segment (start 76.24 106.5) (end 76.24 100.0432) (width 0.2) (layer "F.Cu") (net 1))
 (segment (start 63.8 85.3168) (end 57.5685 91.5483) (width 0.2) (layer "F.Cu") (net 1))
 (segment (start 82.7 92.7) (end 82.7 93.8517) (width 0.2) (layer "F.Cu") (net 1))
 (segment (start 57.3 92.7) (end 57.3 91.5483) (width 0.2) (layer "F.Cu") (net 1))
 (segment (start 96.25 92.25) (end 96.25 98.75) (width 0.2) (layer "F.Cu") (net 1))
 (segment (start 96.25 92.25) (end 95.9483 91.9483) (width 0.2) (layer "F.Cu") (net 1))
 (segment (start 63.8 68.5) (end 63.8 82.8663) (width 0.2) (layer "F.Cu") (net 1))
 (segment (start 92.0588 72.4588) (end 92.0588 80.3412) (width 0.2) (layer "F.Cu") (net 1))
 (segment (start 92.0588 80.3412) (end 90.75 81.65) (width 0.2) (layer "F.Cu") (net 1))
 (segment (start 95.9483 82.9517) (end 97.25 81.65) (width 0.2) (layer "F.Cu") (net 1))
 (segment (start 95.9483 91.9483) (end 95.9483 82.9517) (width 0.2) (layer "F.Cu") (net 1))
 (segment (start 76.24 100.0432) (end 82.4315 93.8517) (width 0.2) (layer "F.Cu") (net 1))
 (segment (start 63.8 82.8663) (end 63.8 85.3168) (width 0.2) (layer "F.Cu") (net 1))
 (segment (start 57.5685 91.5483) (end 57.3 91.5483) (width 0.2) (layer "F.Cu") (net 1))
 (segment (start 90.75 71.15) (end 92.0588 72.4588) (width 0.2) (layer "F.Cu") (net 1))
 (via (at 63.8 82.8663) (size 0.6) (drill 0.3) (layers "F.Cu" "B.Cu") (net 1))
 (segment (start 94.8928 93.6072) (end 96.25 92.25) (width 0.2) (layer "B.Cu") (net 1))
 (segment (start 90.465 81.365) (end 90.75 81.65) (width 0.2) (layer "B.Cu") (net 1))
 (segment (start 63.8 82.8663) (end 65.3013 81.365) (width 0.2) (layer "B.Cu") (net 1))
 (segment (start 82.7 92.7) (end 83.8517 92.7) (width 0.2) (layer "B.Cu") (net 1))
 (segment (start 83.8517 92.7) (end 84.7589 93.6072) (width 0.2) (layer "B.Cu") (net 1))
 (segment (start 90.75 60.65) (end 97.25 60.65) (width 0.2) (layer "B.Cu") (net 1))
 (segment (start 90.75 81.65) (end 97.25 81.65) (width 0.2) (layer "B.Cu") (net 1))
 (segment (start 84.7589 93.6072) (end 94.8928 93.6072) (width 0.2) (layer "B.Cu") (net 1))
 (segment (start 65.3013 81.365) (end 90.465 81.365) (width 0.2) (layer "B.Cu") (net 1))
 (segment (start 90.75 71.15) (end 97.25 71.15) (width 0.2) (layer "B.Cu") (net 1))
 (segment (start 97.81 101.5) (end 97.81 89) (width 0.2) (layer "F.Cu") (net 3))
 (segment (start 98.5625 78.5) (end 98.5625 68.8125) (width 0.2) (layer "F.Cu") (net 3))
 (segment (start 98.5625 68.8125) (end 97.8 68.05) (width 0.2) (layer "F.Cu") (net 3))
 (segment (start 97.81 78.5) (end 98.5625 78.5) (width 0.2) (layer "F.Cu") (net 3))
 (segment (start 97.81 89) (end 98.5625 88.2475) (width 0.2) (layer "F.Cu") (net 3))
 (segment (start 98.5625 88.2475) (end 98.5625 78.5) (width 0.2) (layer "F.Cu") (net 3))
 (segment (start 92.81 106.5) (end 97.81 101.5) (width 0.2) (layer "B.Cu") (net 3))
 (segment (start 89.4494 69.0899) (end 96.7601 69.0899) (width 0.2) (layer "B.Cu") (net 3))
 (segment (start 96.7601 69.0899) (end 97.8 68.05) (width 0.2) (layer "B.Cu") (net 3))
 (segment (start 78.78 106.5) (end 92.81 106.5) (width 0.2) (layer "B.Cu") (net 3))
 (segment (start 76.5 68.5) (end 88.8595 68.5) (width 0.2) (layer "B.Cu") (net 3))
 (segment (start 64.8017 88.89) (end 88.7695 88.89) (width 0.2) (layer "B.Cu") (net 3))
 (segment (start 88.8595 68.5) (end 89.4494 69.0899) (width 0.2) (layer "B.Cu") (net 3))
 (segment (start 57.3 95.24) (end 58.4517 95.24) (width 0.2) (layer "B.Cu") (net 3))
 (segment (start 96.8011 87.9911) (end 97.81 89) (width 0.2) (layer "B.Cu") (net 3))
 (segment (start 58.4517 95.24) (end 64.8017 88.89) (width 0.2) (layer "B.Cu") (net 3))
 (segment (start 89.6684 87.9911) (end 96.8011 87.9911) (width 0.2) (layer "B.Cu") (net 3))
 (segment (start 88.7695 88.89) (end 89.6684 87.9911) (width 0.2) (layer "B.Cu") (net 3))
 (segment (start 61.7168 59.68) (end 70.2683 68.2315) (width 0.2) (layer "B.Cu") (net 18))
 (segment (start 57.3 59.68) (end 61.7168 59.68) (width 0.2) (layer "B.Cu") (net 18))
 (segment (start 71.42 68.5) (end 70.2683 68.5) (width 0.2) (layer "B.Cu") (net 18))
 (segment (start 70.2683 68.2315) (end 70.2683 68.5) (width 0.2) (layer "B.Cu") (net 18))
 (segment (start 73.96 68.5) (end 72.8083 68.5) (width 0.2) (layer "B.Cu") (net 17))
 (segment (start 72.8083 68.7879) (end 64.1362 77.46) (width 0.2) (layer "B.Cu") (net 17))
 (segment (start 72.8083 68.5) (end 72.8083 68.7879) (width 0.2) (layer "B.Cu") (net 17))
 (segment (start 64.1362 77.46) (end 57.3 77.46) (width 0.2) (layer "B.Cu") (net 17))
 (segment (start 67.7283 68.7685) (end 67.7283 68.5) (width 0.2) (layer "B.Cu") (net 19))
 (segment (start 57.3 74.92) (end 61.5768 74.92) (width 0.2) (layer "B.Cu") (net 19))
 (segment (start 68.88 68.5) (end 67.7283 68.5) (width 0.2) (layer "B.Cu") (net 19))
 (segment (start 61.5768 74.92) (end 67.7283 68.7685) (width 0.2) (layer "B.Cu") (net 19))
 (segment (start 63.54 88.3345) (end 63.54 106.5) (width 0.2) (layer "F.Cu") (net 7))
 (segment (start 66.1415 85.733) (end 63.54 88.3345) (width 0.2) (layer "F.Cu") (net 7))
 (via (at 66.1415 85.733) (size 0.6) (drill 0.3) (layers "F.Cu" "B.Cu") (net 7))
 (segment (start 82.7 85.08) (end 66.7945 85.08) (width 0.2) (layer "B.Cu") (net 7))
 (segment (start 66.7945 85.08) (end 66.1415 85.733) (width 0.2) (layer "B.Cu") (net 7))
 (segment (start 66.08 97.2613) (end 66.08 106.5) (width 0.2) (layer "F.Cu") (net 8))
 (segment (start 66.3052 97.0361) (end 66.08 97.2613) (width 0.2) (layer "F.Cu") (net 8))
 (via (at 66.3052 97.0361) (size 0.6) (drill 0.3) (layers "F.Cu" "B.Cu") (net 8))
 (segment (start 66.3052 97.0361) (end 73.1813 90.16) (width 0.2) (layer "B.Cu") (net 8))
 (segment (start 73.1813 90.16) (end 82.7 90.16) (width 0.2) (layer "B.Cu") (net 8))
 (segment (start 68.62 94.9632) (end 82.4315 81.1517) (width 0.2) (layer "F.Cu") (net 9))
 (segment (start 82.4315 81.1517) (end 82.7 81.1517) (width 0.2) (layer "F.Cu") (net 9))
 (segment (start 82.7 80) (end 82.7 81.1517) (width 0.2) (layer "F.Cu") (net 9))
 (segment (start 68.62 106.5) (end 68.62 94.9632) (width 0.2) (layer "F.Cu") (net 9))
 (segment (start 73.1238 95.24) (end 82.7 95.24) (width 0.2) (layer "B.Cu") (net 6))
 (segment (start 62.1517 106.2121) (end 73.1238 95.24) (width 0.2) (layer "B.Cu") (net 6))
 (segment (start 62.1517 106.5) (end 62.1517 106.2121) (width 0.2) (layer "B.Cu") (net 6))
 (segment (start 61 106.5) (end 62.1517 106.5) (width 0.2) (layer "B.Cu") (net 6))
 (segment (start 57.2825 105.7999) (end 56.1457 104.6631) (width 0.2) (layer "F.Cu") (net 11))
 (segment (start 56.1457 104.6631) (end 56.1457 91.3143) (width 0.2) (layer "F.Cu") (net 11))
 (segment (start 57.2825 105.7999) (end 56.1457 104.6631) (width 0.2) (layer "F.Cu") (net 11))
 (segment (start 56.1457 91.3143) (end 57.3 90.16) (width 0.2) (layer "F.Cu") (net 11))
 (segment (start 56.1457 104.6631) (end 57.2825 105.7999) (width 0.2) (layer "F.Cu") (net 11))
 (via (at 57.2825 105.7999) (size 0.6) (drill 0.3) (layers "F.Cu" "B.Cu") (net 11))
 (segment (start 57.2825 105.7999) (end 56.1457 104.6631) (width 0.2) (layer "B.Cu") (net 11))
 (segment (start 73.7 106.5) (end 72.5483 107.6517) (width 0.2) (layer "B.Cu") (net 11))
 (segment (start 72.5483 107.6517) (end 59.1343 107.6517) (width 0.2) (layer "B.Cu") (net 11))
 (segment (start 59.1343 107.6517) (end 57.2825 105.7999) (width 0.2) (layer "B.Cu") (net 11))
 (segment (start 56.1457 104.6631) (end 57.2825 105.7999) (width 0.2) (layer "B.Cu") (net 11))
 (segment (start 82.4121 83.6917) (end 82.7 83.6917) (width 0.2) (layer "F.Cu") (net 10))
 (segment (start 82.7 82.54) (end 82.7 83.6917) (width 0.2) (layer "F.Cu") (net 10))
 (segment (start 71.16 106.5) (end 71.16 94.9438) (width 0.2) (layer "F.Cu") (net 10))
 (segment (start 71.16 94.9438) (end 82.4121 83.6917) (width 0.2) (layer "F.Cu") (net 10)))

